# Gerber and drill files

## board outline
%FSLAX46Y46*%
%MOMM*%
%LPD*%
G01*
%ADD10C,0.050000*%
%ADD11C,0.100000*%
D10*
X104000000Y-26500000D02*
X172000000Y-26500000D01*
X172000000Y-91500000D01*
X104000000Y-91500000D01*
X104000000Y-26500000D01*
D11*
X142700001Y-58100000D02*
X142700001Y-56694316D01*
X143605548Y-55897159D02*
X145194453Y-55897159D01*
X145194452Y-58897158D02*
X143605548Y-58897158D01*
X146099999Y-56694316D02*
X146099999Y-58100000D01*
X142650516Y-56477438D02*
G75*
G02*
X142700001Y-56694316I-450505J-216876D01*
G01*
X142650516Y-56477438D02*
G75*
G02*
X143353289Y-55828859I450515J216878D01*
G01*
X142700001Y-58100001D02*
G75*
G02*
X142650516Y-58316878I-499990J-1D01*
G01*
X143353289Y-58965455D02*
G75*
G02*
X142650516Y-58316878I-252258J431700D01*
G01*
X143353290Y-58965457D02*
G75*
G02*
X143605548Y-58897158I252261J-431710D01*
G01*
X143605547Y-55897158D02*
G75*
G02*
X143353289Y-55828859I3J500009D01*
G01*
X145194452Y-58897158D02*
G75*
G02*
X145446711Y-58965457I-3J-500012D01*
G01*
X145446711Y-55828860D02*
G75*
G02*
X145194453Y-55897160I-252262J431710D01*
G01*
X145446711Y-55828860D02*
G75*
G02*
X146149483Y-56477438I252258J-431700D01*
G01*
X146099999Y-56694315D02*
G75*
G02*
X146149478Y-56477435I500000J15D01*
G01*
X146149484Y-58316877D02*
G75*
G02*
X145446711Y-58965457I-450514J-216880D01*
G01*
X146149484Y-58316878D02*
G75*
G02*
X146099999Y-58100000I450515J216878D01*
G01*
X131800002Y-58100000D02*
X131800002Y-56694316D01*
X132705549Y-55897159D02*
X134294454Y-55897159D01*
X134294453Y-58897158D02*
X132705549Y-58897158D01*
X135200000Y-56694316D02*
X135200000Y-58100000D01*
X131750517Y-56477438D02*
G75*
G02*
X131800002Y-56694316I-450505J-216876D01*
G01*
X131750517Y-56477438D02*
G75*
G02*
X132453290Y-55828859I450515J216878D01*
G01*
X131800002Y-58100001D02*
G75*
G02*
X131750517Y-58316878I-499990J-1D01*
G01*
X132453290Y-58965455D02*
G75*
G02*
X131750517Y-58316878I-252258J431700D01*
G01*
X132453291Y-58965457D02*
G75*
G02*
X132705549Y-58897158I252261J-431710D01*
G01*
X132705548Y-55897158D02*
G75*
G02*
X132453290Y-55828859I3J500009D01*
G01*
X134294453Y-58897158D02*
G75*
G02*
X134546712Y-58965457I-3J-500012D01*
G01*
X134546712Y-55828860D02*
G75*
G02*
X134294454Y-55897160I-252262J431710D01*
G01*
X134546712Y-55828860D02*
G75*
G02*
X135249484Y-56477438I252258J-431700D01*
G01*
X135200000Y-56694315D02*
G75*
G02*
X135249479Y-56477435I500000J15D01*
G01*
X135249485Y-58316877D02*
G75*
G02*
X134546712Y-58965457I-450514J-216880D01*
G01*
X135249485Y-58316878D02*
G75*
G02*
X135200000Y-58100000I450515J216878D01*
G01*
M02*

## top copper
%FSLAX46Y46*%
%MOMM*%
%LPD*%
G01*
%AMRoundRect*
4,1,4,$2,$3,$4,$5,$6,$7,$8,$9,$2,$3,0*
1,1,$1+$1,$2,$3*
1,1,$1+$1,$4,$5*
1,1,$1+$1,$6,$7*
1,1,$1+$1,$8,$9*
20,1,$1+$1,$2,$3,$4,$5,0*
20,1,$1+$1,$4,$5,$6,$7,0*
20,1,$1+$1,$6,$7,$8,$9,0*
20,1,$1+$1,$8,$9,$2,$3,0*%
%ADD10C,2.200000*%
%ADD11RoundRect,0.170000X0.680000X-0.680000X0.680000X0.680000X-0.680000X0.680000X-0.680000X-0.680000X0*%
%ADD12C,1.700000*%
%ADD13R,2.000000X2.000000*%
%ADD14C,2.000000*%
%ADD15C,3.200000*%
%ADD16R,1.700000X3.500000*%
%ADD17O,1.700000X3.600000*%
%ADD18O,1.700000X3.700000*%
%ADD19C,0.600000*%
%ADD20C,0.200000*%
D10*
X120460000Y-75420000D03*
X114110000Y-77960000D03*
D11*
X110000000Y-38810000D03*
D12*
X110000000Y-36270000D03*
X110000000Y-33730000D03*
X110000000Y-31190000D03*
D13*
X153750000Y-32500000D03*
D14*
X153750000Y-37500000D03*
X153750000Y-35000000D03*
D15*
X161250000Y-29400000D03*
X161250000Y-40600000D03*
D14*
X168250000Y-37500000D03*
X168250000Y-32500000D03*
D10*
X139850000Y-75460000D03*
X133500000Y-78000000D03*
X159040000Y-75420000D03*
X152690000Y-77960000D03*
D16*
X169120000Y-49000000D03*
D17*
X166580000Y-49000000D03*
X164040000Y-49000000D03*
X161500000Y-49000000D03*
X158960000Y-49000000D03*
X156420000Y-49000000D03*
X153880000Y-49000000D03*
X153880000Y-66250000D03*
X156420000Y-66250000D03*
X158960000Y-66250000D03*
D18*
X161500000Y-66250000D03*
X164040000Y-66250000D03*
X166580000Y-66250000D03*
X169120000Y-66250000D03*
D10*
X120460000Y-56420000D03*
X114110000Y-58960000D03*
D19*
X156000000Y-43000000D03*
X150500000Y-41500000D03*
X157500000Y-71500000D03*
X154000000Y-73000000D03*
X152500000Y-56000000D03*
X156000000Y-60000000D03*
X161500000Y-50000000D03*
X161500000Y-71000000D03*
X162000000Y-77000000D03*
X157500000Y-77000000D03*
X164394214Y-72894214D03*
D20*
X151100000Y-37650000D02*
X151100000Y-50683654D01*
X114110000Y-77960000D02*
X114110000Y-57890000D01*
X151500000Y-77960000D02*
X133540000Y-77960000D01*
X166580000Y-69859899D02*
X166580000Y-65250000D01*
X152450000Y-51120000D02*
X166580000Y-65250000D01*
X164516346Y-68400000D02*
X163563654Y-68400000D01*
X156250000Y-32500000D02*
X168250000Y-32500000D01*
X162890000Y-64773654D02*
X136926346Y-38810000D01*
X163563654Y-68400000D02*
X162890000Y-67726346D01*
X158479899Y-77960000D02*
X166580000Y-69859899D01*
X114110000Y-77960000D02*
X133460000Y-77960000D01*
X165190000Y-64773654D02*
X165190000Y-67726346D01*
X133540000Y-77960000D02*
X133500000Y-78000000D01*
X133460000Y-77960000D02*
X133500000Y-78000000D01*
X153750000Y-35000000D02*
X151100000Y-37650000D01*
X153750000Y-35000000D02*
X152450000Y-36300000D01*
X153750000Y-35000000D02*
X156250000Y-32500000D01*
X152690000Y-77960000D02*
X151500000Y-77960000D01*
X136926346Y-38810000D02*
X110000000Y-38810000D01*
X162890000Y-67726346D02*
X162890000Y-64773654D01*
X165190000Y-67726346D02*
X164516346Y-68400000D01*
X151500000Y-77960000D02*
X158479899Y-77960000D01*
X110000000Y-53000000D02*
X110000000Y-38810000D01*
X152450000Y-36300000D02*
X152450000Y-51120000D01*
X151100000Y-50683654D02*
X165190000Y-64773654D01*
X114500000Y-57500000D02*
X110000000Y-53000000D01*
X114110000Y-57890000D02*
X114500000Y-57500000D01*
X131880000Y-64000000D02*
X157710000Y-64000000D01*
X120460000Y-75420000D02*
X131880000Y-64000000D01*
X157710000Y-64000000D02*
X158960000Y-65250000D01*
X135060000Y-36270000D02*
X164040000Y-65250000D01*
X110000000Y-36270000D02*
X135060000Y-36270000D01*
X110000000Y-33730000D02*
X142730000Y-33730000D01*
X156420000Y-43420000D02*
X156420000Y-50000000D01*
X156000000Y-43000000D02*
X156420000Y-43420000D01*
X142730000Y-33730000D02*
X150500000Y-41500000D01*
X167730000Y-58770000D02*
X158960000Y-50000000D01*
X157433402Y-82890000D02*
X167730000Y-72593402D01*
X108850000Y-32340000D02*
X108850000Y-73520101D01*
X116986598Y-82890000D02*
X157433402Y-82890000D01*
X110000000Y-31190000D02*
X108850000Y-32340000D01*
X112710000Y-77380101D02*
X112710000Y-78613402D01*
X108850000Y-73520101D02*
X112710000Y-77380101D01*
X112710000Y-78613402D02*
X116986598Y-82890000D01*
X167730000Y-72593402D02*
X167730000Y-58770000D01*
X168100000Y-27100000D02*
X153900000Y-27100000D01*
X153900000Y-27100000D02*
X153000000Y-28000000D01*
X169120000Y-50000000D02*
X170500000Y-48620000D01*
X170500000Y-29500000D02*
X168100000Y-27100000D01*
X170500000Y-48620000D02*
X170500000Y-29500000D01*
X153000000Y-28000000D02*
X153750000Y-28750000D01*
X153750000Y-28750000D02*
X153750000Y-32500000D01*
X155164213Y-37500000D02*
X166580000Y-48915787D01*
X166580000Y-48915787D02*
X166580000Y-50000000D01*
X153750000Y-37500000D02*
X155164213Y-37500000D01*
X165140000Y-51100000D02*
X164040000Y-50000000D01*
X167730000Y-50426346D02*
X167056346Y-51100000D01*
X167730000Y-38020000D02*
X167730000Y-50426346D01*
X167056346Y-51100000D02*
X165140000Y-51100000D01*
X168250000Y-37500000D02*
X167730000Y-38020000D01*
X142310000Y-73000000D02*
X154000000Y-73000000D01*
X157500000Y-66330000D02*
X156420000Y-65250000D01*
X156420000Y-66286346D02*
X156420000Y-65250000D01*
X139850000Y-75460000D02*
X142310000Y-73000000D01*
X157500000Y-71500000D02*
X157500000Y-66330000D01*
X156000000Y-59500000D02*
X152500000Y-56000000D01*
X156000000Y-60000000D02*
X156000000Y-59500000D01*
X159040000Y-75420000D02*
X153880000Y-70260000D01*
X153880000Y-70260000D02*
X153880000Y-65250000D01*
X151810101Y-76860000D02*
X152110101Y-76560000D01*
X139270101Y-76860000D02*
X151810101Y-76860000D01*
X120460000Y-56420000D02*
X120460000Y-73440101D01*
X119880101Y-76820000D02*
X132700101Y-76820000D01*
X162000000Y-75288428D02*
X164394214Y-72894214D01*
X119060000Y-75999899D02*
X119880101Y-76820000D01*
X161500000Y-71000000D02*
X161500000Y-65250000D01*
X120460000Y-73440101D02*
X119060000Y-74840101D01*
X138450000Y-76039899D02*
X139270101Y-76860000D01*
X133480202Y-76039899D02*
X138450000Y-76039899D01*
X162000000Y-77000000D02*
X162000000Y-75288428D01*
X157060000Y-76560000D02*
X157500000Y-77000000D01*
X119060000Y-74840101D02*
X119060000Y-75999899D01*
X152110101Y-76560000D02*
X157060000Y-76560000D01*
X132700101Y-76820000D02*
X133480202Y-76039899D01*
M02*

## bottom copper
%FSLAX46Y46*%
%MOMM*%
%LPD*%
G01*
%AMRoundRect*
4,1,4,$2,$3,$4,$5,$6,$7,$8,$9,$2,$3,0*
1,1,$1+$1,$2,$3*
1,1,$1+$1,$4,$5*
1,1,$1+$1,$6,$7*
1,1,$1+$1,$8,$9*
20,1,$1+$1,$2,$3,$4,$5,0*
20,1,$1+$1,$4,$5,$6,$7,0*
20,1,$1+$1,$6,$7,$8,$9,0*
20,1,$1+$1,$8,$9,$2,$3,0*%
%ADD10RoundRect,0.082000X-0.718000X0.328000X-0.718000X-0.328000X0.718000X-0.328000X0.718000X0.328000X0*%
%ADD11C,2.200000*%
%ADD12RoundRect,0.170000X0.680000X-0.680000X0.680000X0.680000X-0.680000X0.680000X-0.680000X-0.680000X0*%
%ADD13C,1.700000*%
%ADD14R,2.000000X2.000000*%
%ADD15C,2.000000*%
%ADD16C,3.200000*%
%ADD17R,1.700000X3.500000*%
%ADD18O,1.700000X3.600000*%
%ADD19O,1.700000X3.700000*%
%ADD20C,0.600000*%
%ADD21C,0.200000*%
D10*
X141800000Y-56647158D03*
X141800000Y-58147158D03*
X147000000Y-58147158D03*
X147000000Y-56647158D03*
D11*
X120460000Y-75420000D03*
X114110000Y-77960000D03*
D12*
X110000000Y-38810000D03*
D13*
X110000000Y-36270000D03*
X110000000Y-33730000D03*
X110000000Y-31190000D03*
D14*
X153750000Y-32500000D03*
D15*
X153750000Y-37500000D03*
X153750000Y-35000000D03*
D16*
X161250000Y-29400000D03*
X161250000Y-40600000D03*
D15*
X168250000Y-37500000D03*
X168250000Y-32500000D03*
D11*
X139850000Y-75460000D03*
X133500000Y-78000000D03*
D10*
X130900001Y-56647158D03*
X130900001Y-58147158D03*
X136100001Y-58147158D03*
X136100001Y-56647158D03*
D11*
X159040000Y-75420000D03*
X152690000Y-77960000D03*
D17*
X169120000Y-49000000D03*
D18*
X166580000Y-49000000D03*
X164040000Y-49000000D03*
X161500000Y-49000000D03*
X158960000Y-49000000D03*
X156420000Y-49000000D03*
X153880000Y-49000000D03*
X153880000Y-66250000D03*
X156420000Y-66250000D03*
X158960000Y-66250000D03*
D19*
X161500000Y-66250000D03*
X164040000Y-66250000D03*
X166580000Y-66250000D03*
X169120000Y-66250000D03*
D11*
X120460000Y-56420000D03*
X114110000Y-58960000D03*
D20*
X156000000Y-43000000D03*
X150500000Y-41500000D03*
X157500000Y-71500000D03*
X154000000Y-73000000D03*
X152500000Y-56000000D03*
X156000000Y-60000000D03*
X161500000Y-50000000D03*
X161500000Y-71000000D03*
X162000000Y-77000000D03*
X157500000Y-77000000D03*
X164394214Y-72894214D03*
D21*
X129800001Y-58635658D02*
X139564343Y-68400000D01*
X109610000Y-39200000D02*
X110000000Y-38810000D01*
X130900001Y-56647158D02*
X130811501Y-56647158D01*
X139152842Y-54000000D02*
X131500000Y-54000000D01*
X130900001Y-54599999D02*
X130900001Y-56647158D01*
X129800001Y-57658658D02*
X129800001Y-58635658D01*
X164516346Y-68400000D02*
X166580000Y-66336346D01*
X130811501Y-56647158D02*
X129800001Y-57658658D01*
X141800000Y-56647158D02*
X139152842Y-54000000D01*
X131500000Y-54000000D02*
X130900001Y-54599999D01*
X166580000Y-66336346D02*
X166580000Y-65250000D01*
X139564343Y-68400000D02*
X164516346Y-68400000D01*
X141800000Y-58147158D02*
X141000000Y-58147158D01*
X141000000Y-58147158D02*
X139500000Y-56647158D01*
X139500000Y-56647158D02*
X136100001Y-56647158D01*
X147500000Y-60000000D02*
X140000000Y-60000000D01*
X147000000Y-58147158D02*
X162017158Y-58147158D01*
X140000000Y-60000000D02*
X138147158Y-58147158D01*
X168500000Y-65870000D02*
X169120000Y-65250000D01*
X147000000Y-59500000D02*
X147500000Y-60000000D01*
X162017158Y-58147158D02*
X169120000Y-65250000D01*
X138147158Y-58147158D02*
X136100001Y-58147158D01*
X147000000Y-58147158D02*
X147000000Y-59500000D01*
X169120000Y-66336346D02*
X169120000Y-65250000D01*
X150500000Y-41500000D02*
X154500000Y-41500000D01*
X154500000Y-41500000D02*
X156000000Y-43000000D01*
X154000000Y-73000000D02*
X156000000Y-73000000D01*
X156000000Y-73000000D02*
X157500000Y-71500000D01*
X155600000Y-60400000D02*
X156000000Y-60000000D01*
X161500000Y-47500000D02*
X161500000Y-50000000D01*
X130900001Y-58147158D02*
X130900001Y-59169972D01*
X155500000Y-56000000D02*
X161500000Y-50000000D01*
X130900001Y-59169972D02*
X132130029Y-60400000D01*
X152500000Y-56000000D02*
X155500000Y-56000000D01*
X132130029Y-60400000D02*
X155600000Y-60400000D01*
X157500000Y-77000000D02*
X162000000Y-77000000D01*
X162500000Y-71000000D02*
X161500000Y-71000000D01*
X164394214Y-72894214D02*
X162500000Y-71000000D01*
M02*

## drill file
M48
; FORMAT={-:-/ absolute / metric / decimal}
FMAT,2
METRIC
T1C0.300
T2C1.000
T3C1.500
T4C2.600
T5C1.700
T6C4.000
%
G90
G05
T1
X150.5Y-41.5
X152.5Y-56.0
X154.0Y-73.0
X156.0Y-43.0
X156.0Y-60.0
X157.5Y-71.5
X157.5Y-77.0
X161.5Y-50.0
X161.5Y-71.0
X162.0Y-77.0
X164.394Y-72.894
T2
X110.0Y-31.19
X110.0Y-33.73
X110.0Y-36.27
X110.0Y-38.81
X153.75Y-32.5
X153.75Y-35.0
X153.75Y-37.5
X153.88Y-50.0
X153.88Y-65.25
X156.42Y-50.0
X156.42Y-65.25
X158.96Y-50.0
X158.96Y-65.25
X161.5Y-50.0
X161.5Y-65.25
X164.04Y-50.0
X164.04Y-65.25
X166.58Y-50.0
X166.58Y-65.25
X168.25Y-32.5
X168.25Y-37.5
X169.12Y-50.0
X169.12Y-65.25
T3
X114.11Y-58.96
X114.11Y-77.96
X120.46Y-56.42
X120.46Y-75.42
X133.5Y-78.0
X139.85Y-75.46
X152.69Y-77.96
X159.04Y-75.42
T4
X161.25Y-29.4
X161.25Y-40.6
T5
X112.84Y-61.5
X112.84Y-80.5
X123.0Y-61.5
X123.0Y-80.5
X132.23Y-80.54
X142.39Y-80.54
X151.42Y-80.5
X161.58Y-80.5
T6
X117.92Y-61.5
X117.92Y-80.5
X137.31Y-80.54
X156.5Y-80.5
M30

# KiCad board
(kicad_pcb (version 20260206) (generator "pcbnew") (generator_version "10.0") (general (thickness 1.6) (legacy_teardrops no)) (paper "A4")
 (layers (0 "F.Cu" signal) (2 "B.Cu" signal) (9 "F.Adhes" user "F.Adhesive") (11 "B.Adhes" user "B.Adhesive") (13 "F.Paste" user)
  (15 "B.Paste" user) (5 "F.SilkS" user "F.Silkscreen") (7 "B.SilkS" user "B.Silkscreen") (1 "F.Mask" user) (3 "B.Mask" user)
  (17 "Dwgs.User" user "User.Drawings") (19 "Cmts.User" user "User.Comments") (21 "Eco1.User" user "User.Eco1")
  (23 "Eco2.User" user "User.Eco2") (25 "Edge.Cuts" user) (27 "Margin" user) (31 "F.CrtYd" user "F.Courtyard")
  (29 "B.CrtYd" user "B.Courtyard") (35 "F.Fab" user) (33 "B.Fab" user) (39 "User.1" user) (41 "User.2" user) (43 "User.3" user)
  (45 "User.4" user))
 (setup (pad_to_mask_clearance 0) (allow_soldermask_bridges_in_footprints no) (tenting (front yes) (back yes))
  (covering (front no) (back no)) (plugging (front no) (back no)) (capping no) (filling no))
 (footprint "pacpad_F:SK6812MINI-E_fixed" (layer "F.Cu") (at 144.399999 57.5)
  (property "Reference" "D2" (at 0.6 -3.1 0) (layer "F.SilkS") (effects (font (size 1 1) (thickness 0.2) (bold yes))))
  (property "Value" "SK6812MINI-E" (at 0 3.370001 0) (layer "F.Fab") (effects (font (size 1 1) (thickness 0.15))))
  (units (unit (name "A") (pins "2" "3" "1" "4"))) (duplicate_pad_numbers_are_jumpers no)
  (fp_line (start -1.699998 0.6) (end -1.699998 -0.805684) (stroke (width 0.1) (type solid)) (layer "Edge.Cuts"))
  (fp_line (start -0.794451 -1.602841) (end 0.794454 -1.602841) (stroke (width 0.1) (type solid)) (layer "Edge.Cuts"))
  (fp_line (start 0.794453 1.397158) (end -0.794451 1.397158) (stroke (width 0.1) (type solid)) (layer "Edge.Cuts"))
  (fp_line (start 1.7 -0.805684) (end 1.7 0.6) (stroke (width 0.1) (type solid)) (layer "Edge.Cuts"))
  (fp_arc (start -1.749483 -1.022562) (mid -1.712526 -0.91691) (end -1.699998 -0.805684) (stroke (width 0.1) (type solid))
   (layer "Edge.Cuts"))
  (fp_arc (start -1.749483 -1.022562) (mid -1.63807 -1.606877) (end -1.04671 -1.671141) (stroke (width 0.1) (type solid))
   (layer "Edge.Cuts"))
  (fp_arc (start -1.699998 0.600001) (mid -1.712526 0.711226) (end -1.749483 0.816878) (stroke (width 0.1) (type solid)) (layer "Edge.Cuts"))
  (fp_arc (start -1.04671 1.465455) (mid -1.638069 1.401192) (end -1.749483 0.816878) (stroke (width 0.1) (type solid)) (layer "Edge.Cuts"))
  (fp_arc (start -1.046709 1.465457) (mid -0.925121 1.414535) (end -0.794451 1.397158) (stroke (width 0.1) (type solid)) (layer "Edge.Cuts"))
  (fp_arc (start -0.794452 -1.602842) (mid -0.925122 -1.620219) (end -1.04671 -1.671141) (stroke (width 0.1) (type solid))
   (layer "Edge.Cuts"))
  (fp_arc (start 0.794453 1.397158) (mid 0.925124 1.414535) (end 1.046712 1.465457) (stroke (width 0.1) (type solid)) (layer "Edge.Cuts"))
  (fp_arc (start 1.046712 -1.67114) (mid 0.925124 -1.620218) (end 0.794454 -1.602841) (stroke (width 0.1) (type solid)) (layer "Edge.Cuts"))
  (fp_arc (start 1.046712 -1.67114) (mid 1.638072 -1.606876) (end 1.749485 -1.022562) (stroke (width 0.1) (type solid)) (layer "Edge.Cuts"))
  (fp_arc (start 1.7 -0.805685) (mid 1.712528 -0.91691) (end 1.749485 -1.022562) (stroke (width 0.1) (type solid)) (layer "Edge.Cuts"))
  (fp_arc (start 1.749485 0.816877) (mid 1.638073 1.401193) (end 1.046712 1.465457) (stroke (width 0.1) (type solid)) (layer "Edge.Cuts"))
  (fp_arc (start 1.749485 0.816878) (mid 1.712528 0.711226) (end 1.7 0.6) (stroke (width 0.1) (type solid)) (layer "Edge.Cuts"))
  (pad "1" smd roundrect (at -2.599999 -0.852842 270) (size 0.82 1.6) (layers "B.Cu" "B.Mask" "B.Paste") (roundrect_rratio 0.1) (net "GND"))
  (pad "2" smd roundrect (at -2.599999 0.647158 270) (size 0.82 1.6) (layers "B.Cu" "B.Mask" "B.Paste") (roundrect_rratio 0.1)
   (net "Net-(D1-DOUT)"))
  (pad "3" smd roundrect (at 2.600001 0.647158 270) (size 0.82 1.6) (layers "B.Cu" "B.Mask" "B.Paste") (roundrect_rratio 0.1)
   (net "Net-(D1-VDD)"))
  (pad "4" smd roundrect (at 2.600001 -0.852842 270) (size 0.82 1.6) (layers "B.Cu" "B.Mask" "B.Paste") (roundrect_rratio 0.1)
   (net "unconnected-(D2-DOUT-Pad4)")))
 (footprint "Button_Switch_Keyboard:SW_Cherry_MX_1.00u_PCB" (layer "F.Cu") (at 120.46 75.42)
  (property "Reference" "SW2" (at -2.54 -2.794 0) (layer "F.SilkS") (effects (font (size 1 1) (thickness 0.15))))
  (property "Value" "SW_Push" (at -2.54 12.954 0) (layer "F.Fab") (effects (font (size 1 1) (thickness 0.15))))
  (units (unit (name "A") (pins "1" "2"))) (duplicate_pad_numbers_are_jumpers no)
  (pad "" np_thru_hole circle (at -7.62 5.08) (size 1.7 1.7) (drill 1.7) (layers "*.Cu" "*.Mask"))
  (pad "" np_thru_hole circle (at -2.54 5.08) (size 4 4) (drill 4) (layers "*.Cu" "*.Mask"))
  (pad "" np_thru_hole circle (at 2.54 5.08) (size 1.7 1.7) (drill 1.7) (layers "*.Cu" "*.Mask"))
  (pad "1" thru_hole circle (at 0 0) (size 2.2 2.2) (drill 1.5) (layers "*.Cu" "*.Mask") (remove_unused_layers no)
   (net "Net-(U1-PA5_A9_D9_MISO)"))
  (pad "2" thru_hole circle (at -6.35 2.54) (size 2.2 2.2) (drill 1.5) (layers "*.Cu" "*.Mask") (remove_unused_layers no) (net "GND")))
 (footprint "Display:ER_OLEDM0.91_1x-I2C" (layer "F.Cu") (at 110 38.81 90)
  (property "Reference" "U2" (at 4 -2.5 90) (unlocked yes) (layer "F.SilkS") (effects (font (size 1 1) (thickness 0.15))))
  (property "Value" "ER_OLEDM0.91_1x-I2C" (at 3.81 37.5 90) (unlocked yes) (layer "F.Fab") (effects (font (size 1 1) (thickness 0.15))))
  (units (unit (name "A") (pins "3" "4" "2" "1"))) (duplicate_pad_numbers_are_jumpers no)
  (pad "1" thru_hole roundrect (at 0 0 90) (size 1.7 1.7) (drill 1) (layers "*.Cu" "*.Mask") (remove_unused_layers no)
   (roundrect_rratio 0.1) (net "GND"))
  (pad "2" thru_hole circle (at 2.54 0 90) (size 1.7 1.7) (drill 1) (layers "*.Cu" "*.Mask") (remove_unused_layers no) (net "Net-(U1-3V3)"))
  (pad "3" thru_hole circle (at 5.08 0 90) (size 1.7 1.7) (drill 1) (layers "*.Cu" "*.Mask") (remove_unused_layers no)
   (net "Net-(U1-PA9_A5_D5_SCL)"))
  (pad "4" thru_hole circle (at 7.62 0 90) (size 1.7 1.7) (drill 1) (layers "*.Cu" "*.Mask") (remove_unused_layers no)
   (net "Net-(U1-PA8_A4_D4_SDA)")))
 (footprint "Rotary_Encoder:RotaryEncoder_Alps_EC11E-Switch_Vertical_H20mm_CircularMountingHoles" (layer "F.Cu") (at 153.75 32.5)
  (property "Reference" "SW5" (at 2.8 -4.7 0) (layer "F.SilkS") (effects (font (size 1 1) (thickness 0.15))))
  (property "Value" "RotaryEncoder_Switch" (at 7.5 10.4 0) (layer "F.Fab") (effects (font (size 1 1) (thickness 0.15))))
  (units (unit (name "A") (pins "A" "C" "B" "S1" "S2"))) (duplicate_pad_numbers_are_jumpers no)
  (pad "A" thru_hole rect (at 0 0) (size 2 2) (drill 1) (layers "*.Cu" "*.Mask") (remove_unused_layers no) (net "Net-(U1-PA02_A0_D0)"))
  (pad "B" thru_hole circle (at 0 5) (size 2 2) (drill 1) (layers "*.Cu" "*.Mask") (remove_unused_layers no) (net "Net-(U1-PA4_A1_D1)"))
  (pad "C" thru_hole circle (at 0 2.5) (size 2 2) (drill 1) (layers "*.Cu" "*.Mask") (remove_unused_layers no) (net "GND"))
  (pad "MP" thru_hole circle (at 7.5 -3.1) (size 3.2 3.2) (drill 2.6) (layers "*.Cu" "*.Mask") (remove_unused_layers no))
  (pad "MP" thru_hole circle (at 7.5 8.1) (size 3.2 3.2) (drill 2.6) (layers "*.Cu" "*.Mask") (remove_unused_layers no))
  (pad "S1" thru_hole circle (at 14.5 5) (size 2 2) (drill 1) (layers "*.Cu" "*.Mask") (remove_unused_layers no) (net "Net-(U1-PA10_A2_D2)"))
  (pad "S2" thru_hole circle (at 14.5 0) (size 2 2) (drill 1) (layers "*.Cu" "*.Mask") (remove_unused_layers no) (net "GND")))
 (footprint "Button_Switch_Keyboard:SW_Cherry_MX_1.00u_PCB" (layer "F.Cu") (at 139.85 75.46)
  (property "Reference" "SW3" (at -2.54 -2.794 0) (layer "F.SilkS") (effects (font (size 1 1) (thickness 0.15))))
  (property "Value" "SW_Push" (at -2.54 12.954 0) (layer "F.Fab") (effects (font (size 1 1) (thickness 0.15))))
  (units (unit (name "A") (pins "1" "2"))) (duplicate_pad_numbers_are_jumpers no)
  (pad "" np_thru_hole circle (at -7.62 5.08) (size 1.7 1.7) (drill 1.7) (layers "*.Cu" "*.Mask"))
  (pad "" np_thru_hole circle (at -2.54 5.08) (size 4 4) (drill 4) (layers "*.Cu" "*.Mask"))
  (pad "" np_thru_hole circle (at 2.54 5.08) (size 1.7 1.7) (drill 1.7) (layers "*.Cu" "*.Mask"))
  (pad "1" thru_hole circle (at 0 0) (size 2.2 2.2) (drill 1.5) (layers "*.Cu" "*.Mask") (remove_unused_layers no)
   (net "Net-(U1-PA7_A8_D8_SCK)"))
  (pad "2" thru_hole circle (at -6.35 2.54) (size 2.2 2.2) (drill 1.5) (layers "*.Cu" "*.Mask") (remove_unused_layers no) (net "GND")))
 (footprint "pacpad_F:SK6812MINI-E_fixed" (layer "F.Cu") (at 133.5 57.5)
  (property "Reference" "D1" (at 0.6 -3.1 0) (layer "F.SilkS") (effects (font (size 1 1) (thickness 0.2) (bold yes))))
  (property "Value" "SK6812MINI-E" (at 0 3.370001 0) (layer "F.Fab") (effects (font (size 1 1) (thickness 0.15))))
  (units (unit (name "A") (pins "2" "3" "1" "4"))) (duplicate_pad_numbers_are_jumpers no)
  (fp_line (start -1.699998 0.6) (end -1.699998 -0.805684) (stroke (width 0.1) (type solid)) (layer "Edge.Cuts"))
  (fp_line (start -0.794451 -1.602841) (end 0.794454 -1.602841) (stroke (width 0.1) (type solid)) (layer "Edge.Cuts"))
  (fp_line (start 0.794453 1.397158) (end -0.794451 1.397158) (stroke (width 0.1) (type solid)) (layer "Edge.Cuts"))
  (fp_line (start 1.7 -0.805684) (end 1.7 0.6) (stroke (width 0.1) (type solid)) (layer "Edge.Cuts"))
  (fp_arc (start -1.749483 -1.022562) (mid -1.712526 -0.91691) (end -1.699998 -0.805684) (stroke (width 0.1) (type solid))
   (layer "Edge.Cuts"))
  (fp_arc (start -1.749483 -1.022562) (mid -1.63807 -1.606877) (end -1.04671 -1.671141) (stroke (width 0.1) (type solid))
   (layer "Edge.Cuts"))
  (fp_arc (start -1.699998 0.600001) (mid -1.712526 0.711226) (end -1.749483 0.816878) (stroke (width 0.1) (type solid)) (layer "Edge.Cuts"))
  (fp_arc (start -1.04671 1.465455) (mid -1.638069 1.401192) (end -1.749483 0.816878) (stroke (width 0.1) (type solid)) (layer "Edge.Cuts"))
  (fp_arc (start -1.046709 1.465457) (mid -0.925121 1.414535) (end -0.794451 1.397158) (stroke (width 0.1) (type solid)) (layer "Edge.Cuts"))
  (fp_arc (start -0.794452 -1.602842) (mid -0.925122 -1.620219) (end -1.04671 -1.671141) (stroke (width 0.1) (type solid))
   (layer "Edge.Cuts"))
  (fp_arc (start 0.794453 1.397158) (mid 0.925124 1.414535) (end 1.046712 1.465457) (stroke (width 0.1) (type solid)) (layer "Edge.Cuts"))
  (fp_arc (start 1.046712 -1.67114) (mid 0.925124 -1.620218) (end 0.794454 -1.602841) (stroke (width 0.1) (type solid)) (layer "Edge.Cuts"))
  (fp_arc (start 1.046712 -1.67114) (mid 1.638072 -1.606876) (end 1.749485 -1.022562) (stroke (width 0.1) (type solid)) (layer "Edge.Cuts"))
  (fp_arc (start 1.7 -0.805685) (mid 1.712528 -0.91691) (end 1.749485 -1.022562) (stroke (width 0.1) (type solid)) (layer "Edge.Cuts"))
  (fp_arc (start 1.749485 0.816877) (mid 1.638073 1.401193) (end 1.046712 1.465457) (stroke (width 0.1) (type solid)) (layer "Edge.Cuts"))
  (fp_arc (start 1.749485 0.816878) (mid 1.712528 0.711226) (end 1.7 0.6) (stroke (width 0.1) (type solid)) (layer "Edge.Cuts"))
  (pad "1" smd roundrect (at -2.599999 -0.852842 270) (size 0.82 1.6) (layers "B.Cu" "B.Mask" "B.Paste") (roundrect_rratio 0.1) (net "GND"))
  (pad "2" smd roundrect (at -2.599999 0.647158 270) (size 0.82 1.6) (layers "B.Cu" "B.Mask" "B.Paste") (roundrect_rratio 0.1)
   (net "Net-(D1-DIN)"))
  (pad "3" smd roundrect (at 2.600001 0.647158 270) (size 0.82 1.6) (layers "B.Cu" "B.Mask" "B.Paste") (roundrect_rratio 0.1)
   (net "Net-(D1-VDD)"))
  (pad "4" smd roundrect (at 2.600001 -0.852842 270) (size 0.82 1.6) (layers "B.Cu" "B.Mask" "B.Paste") (roundrect_rratio 0.1)
   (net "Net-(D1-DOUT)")))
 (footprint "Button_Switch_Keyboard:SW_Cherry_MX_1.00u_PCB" (layer "F.Cu") (at 159.04 75.42)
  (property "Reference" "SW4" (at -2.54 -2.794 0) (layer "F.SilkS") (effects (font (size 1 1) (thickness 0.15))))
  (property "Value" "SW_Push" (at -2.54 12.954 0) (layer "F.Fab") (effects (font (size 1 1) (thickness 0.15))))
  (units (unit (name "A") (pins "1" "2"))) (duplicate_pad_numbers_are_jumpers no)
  (pad "" np_thru_hole circle (at -7.62 5.08) (size 1.7 1.7) (drill 1.7) (layers "*.Cu" "*.Mask"))
  (pad "" np_thru_hole circle (at -2.54 5.08) (size 4 4) (drill 4) (layers "*.Cu" "*.Mask"))
  (pad "" np_thru_hole circle (at 2.54 5.08) (size 1.7 1.7) (drill 1.7) (layers "*.Cu" "*.Mask"))
  (pad "1" thru_hole circle (at 0 0) (size 2.2 2.2) (drill 1.5) (layers "*.Cu" "*.Mask") (remove_unused_layers no)
   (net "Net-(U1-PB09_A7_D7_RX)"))
  (pad "2" thru_hole circle (at -6.35 2.54) (size 2.2 2.2) (drill 1.5) (layers "*.Cu" "*.Mask") (remove_unused_layers no) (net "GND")))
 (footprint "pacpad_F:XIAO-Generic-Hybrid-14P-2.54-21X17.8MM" (layer "F.Cu") (at 161.5 57.625 -90)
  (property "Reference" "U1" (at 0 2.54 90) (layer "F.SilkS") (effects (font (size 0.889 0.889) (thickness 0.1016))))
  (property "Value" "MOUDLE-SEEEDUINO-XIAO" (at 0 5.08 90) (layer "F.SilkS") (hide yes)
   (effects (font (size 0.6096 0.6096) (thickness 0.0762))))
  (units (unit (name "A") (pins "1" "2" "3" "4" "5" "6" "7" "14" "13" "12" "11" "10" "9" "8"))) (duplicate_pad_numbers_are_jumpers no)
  (pad "1" thru_hole rect (at -7.625 -7.62 270) (size 3.5 1.7) (drill 1 (offset -1 0)) (layers "*.Cu" "*.Mask") (remove_unused_layers no)
   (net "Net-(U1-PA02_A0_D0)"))
  (pad "2" thru_hole oval (at -7.625 -5.08 270) (size 3.6 1.7) (drill 1 (offset -1 0)) (layers "*.Cu" "*.Mask") (remove_unused_layers no)
   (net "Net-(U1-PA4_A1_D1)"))
  (pad "3" thru_hole oval (at -7.625 -2.54 270) (size 3.6 1.7) (drill 1 (offset -1 0)) (layers "*.Cu" "*.Mask") (remove_unused_layers no)
   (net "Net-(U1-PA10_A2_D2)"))
  (pad "4" thru_hole oval (at -7.625 0 270) (size 3.6 1.7) (drill 1 (offset -1 0)) (layers "*.Cu" "*.Mask") (remove_unused_layers no)
   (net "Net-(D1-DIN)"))
  (pad "5" thru_hole oval (at -7.625 2.54 270) (size 3.6 1.7) (drill 1 (offset -1 0)) (layers "*.Cu" "*.Mask") (remove_unused_layers no)
   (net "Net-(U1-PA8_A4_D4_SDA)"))
  (pad "6" thru_hole oval (at -7.625 5.08 90) (size 3.6 1.7) (drill 1 (offset 1 0)) (layers "*.Cu" "*.Mask") (remove_unused_layers no)
   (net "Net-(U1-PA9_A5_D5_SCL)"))
  (pad "7" thru_hole oval (at -7.625 7.62 270) (size 3.6 1.7) (drill 1 (offset -1 0)) (layers "*.Cu" "*.Mask") (remove_unused_layers no)
   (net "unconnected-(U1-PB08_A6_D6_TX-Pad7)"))
  (pad "8" thru_hole oval (at 7.625 7.62 270) (size 3.6 1.7) (drill 1 (offset 1 0)) (layers "*.Cu" "*.Mask") (remove_unused_layers no)
   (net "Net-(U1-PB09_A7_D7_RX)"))
  (pad "9" thru_hole oval (at 7.625 5.08 270) (size 3.6 1.7) (drill 1 (offset 1 0)) (layers "*.Cu" "*.Mask") (remove_unused_layers no)
   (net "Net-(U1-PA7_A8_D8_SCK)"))
  (pad "10" thru_hole oval (at 7.625 2.54 270) (size 3.6 1.7) (drill 1 (offset 1 0)) (layers "*.Cu" "*.Mask") (remove_unused_layers no)
   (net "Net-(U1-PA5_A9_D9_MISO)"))
  (pad "11" thru_hole oval (at 7.625 0 270) (size 3.7 1.7) (drill 1 (offset 1 0)) (layers "*.Cu" "*.Mask") (remove_unused_layers no)
   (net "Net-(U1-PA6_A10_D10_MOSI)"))
  (pad "12" thru_hole oval (at 7.625 -2.54 270) (size 3.7 1.7) (drill 1 (offset 1 0)) (layers "*.Cu" "*.Mask") (remove_unused_layers no)
   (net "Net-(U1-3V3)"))
  (pad "13" thru_hole oval (at 7.625 -5.08 270) (size 3.7 1.7) (drill 1 (offset 1 0)) (layers "*.Cu" "*.Mask") (remove_unused_layers no)
   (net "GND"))
  (pad "14" thru_hole oval (at 7.625 -7.62 270) (size 3.7 1.7) (drill 1 (offset 1 0)) (layers "*.Cu" "*.Mask") (remove_unused_layers no)
   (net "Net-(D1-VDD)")))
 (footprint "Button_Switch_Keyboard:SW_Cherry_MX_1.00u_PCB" (layer "F.Cu") (at 120.46 56.42)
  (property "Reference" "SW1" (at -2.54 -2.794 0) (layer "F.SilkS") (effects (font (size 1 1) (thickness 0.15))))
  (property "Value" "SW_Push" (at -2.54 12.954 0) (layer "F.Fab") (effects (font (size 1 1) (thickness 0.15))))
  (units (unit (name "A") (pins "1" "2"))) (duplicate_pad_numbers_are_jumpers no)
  (pad "" np_thru_hole circle (at -7.62 5.08) (size 1.7 1.7) (drill 1.7) (layers "*.Cu" "*.Mask"))
  (pad "" np_thru_hole circle (at -2.54 5.08) (size 4 4) (drill 4) (layers "*.Cu" "*.Mask"))
  (pad "" np_thru_hole circle (at 2.54 5.08) (size 1.7 1.7) (drill 1.7) (layers "*.Cu" "*.Mask"))
  (pad "1" thru_hole circle (at 0 0) (size 2.2 2.2) (drill 1.5) (layers "*.Cu" "*.Mask") (remove_unused_layers no)
   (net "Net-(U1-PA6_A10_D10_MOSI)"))
  (pad "2" thru_hole circle (at -6.35 2.54) (size 2.2 2.2) (drill 1.5) (layers "*.Cu" "*.Mask") (remove_unused_layers no) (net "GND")))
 (gr_rect (start 104 26.5) (end 172 91.5) (stroke (width 0.05) (type default)) (fill no) (layer "Edge.Cuts"))
 (segment (start 151.1 37.65) (end 151.1 50.683654) (width 0.2) (layer "F.Cu") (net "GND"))
 (segment (start 114.11 77.96) (end 114.11 57.89) (width 0.2) (layer "F.Cu") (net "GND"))
 (segment (start 151.5 77.96) (end 133.54 77.96) (width 0.2) (layer "F.Cu") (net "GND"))
 (segment (start 166.58 69.859899) (end 166.58 65.25) (width 0.2) (layer "F.Cu") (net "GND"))
 (segment (start 152.45 51.12) (end 166.58 65.25) (width 0.2) (layer "F.Cu") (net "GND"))
 (segment (start 164.516346 68.4) (end 163.563654 68.4) (width 0.2) (layer "F.Cu") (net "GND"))
 (segment (start 156.25 32.5) (end 168.25 32.5) (width 0.2) (layer "F.Cu") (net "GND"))
 (segment (start 162.89 64.773654) (end 136.926346 38.81) (width 0.2) (layer "F.Cu") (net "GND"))
 (segment (start 163.563654 68.4) (end 162.89 67.726346) (width 0.2) (layer "F.Cu") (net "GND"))
 (segment (start 158.479899 77.96) (end 166.58 69.859899) (width 0.2) (layer "F.Cu") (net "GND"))
 (segment (start 114.11 77.96) (end 133.46 77.96) (width 0.2) (layer "F.Cu") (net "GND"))
 (segment (start 165.19 64.773654) (end 165.19 67.726346) (width 0.2) (layer "F.Cu") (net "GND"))
 (segment (start 133.54 77.96) (end 133.5 78) (width 0.2) (layer "F.Cu") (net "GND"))
 (segment (start 133.46 77.96) (end 133.5 78) (width 0.2) (layer "F.Cu") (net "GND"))
 (segment (start 153.75 35) (end 151.1 37.65) (width 0.2) (layer "F.Cu") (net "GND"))
 (segment (start 153.75 35) (end 152.45 36.3) (width 0.2) (layer "F.Cu") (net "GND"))
 (segment (start 153.75 35) (end 156.25 32.5) (width 0.2) (layer "F.Cu") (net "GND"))
 (segment (start 152.69 77.96) (end 151.5 77.96) (width 0.2) (layer "F.Cu") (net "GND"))
 (segment (start 136.926346 38.81) (end 110 38.81) (width 0.2) (layer "F.Cu") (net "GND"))
 (segment (start 162.89 67.726346) (end 162.89 64.773654) (width 0.2) (layer "F.Cu") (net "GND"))
 (segment (start 165.19 67.726346) (end 164.516346 68.4) (width 0.2) (layer "F.Cu") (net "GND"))
 (segment (start 151.5 77.96) (end 158.479899 77.96) (width 0.2) (layer "F.Cu") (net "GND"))
 (segment (start 110 53) (end 110 38.81) (width 0.2) (layer "F.Cu") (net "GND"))
 (segment (start 152.45 36.3) (end 152.45 51.12) (width 0.2) (layer "F.Cu") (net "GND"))
 (segment (start 151.1 50.683654) (end 165.19 64.773654) (width 0.2) (layer "F.Cu") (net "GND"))
 (segment (start 114.5 57.5) (end 110 53) (width 0.2) (layer "F.Cu") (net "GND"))
 (segment (start 114.11 57.89) (end 114.5 57.5) (width 0.2) (layer "F.Cu") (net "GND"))
 (segment (start 129.800001 58.635658) (end 139.564343 68.4) (width 0.2) (layer "B.Cu") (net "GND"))
 (segment (start 109.61 39.2) (end 110 38.81) (width 0.2) (layer "B.Cu") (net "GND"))
 (segment (start 130.900001 56.647158) (end 130.811501 56.647158) (width 0.2) (layer "B.Cu") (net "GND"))
 (segment (start 139.152842 54) (end 131.5 54) (width 0.2) (layer "B.Cu") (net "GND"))
 (segment (start 130.900001 54.599999) (end 130.900001 56.647158) (width 0.2) (layer "B.Cu") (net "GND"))
 (segment (start 129.800001 57.658658) (end 129.800001 58.635658) (width 0.2) (layer "B.Cu") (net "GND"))
 (segment (start 164.516346 68.4) (end 166.58 66.336346) (width 0.2) (layer "B.Cu") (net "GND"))
 (segment (start 130.811501 56.647158) (end 129.800001 57.658658) (width 0.2) (layer "B.Cu") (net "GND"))
 (segment (start 141.8 56.647158) (end 139.152842 54) (width 0.2) (layer "B.Cu") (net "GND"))
 (segment (start 131.5 54) (end 130.900001 54.599999) (width 0.2) (layer "B.Cu") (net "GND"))
 (segment (start 166.58 66.336346) (end 166.58 65.25) (width 0.2) (layer "B.Cu") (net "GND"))
 (segment (start 139.564343 68.4) (end 164.516346 68.4) (width 0.2) (layer "B.Cu") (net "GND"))
 (segment (start 141.8 58.147158) (end 141 58.147158) (width 0.2) (layer "B.Cu") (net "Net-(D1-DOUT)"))
 (segment (start 141 58.147158) (end 139.5 56.647158) (width 0.2) (layer "B.Cu") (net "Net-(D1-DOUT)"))
 (segment (start 139.5 56.647158) (end 136.100001 56.647158) (width 0.2) (layer "B.Cu") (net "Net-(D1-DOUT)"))
 (segment (start 147.5 60) (end 140 60) (width 0.2) (layer "B.Cu") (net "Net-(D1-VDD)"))
 (segment (start 147 58.147158) (end 162.017158 58.147158) (width 0.2) (layer "B.Cu") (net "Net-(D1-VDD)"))
 (segment (start 140 60) (end 138.147158 58.147158) (width 0.2) (layer "B.Cu") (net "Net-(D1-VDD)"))
 (segment (start 168.5 65.87) (end 169.12 65.25) (width 0.2) (layer "B.Cu") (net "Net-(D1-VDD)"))
 (segment (start 147 59.5) (end 147.5 60) (width 0.2) (layer "B.Cu") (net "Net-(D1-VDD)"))
 (segment (start 162.017158 58.147158) (end 169.12 65.25) (width 0.2) (layer "B.Cu") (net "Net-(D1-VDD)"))
 (segment (start 138.147158 58.147158) (end 136.100001 58.147158) (width 0.2) (layer "B.Cu") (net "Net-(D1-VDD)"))
 (segment (start 147 58.147158) (end 147 59.5) (width 0.2) (layer "B.Cu") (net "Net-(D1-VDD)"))
 (segment (start 169.12 66.336346) (end 169.12 65.25) (width 0.2) (layer "B.Cu") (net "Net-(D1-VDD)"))
 (segment (start 131.88 64) (end 157.71 64) (width 0.2) (layer "F.Cu") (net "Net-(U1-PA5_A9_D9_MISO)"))
 (segment (start 120.46 75.42) (end 131.88 64) (width 0.2) (layer "F.Cu") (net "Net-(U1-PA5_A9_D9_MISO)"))
 (segment (start 157.71 64) (end 158.96 65.25) (width 0.2) (layer "F.Cu") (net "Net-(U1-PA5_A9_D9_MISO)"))
 (segment (start 135.06 36.27) (end 164.04 65.25) (width 0.2) (layer "F.Cu") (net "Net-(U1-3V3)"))
 (segment (start 110 36.27) (end 135.06 36.27) (width 0.2) (layer "F.Cu") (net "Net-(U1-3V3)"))
 (segment (start 110 33.73) (end 142.73 33.73) (width 0.2) (layer "F.Cu") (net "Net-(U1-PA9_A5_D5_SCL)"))
 (segment (start 156.42 43.42) (end 156.42 50) (width 0.2) (layer "F.Cu") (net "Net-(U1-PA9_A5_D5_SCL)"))
 (segment (start 156 43) (end 156.42 43.42) (width 0.2) (layer "F.Cu") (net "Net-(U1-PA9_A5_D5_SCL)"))
 (segment (start 142.73 33.73) (end 150.5 41.5) (width 0.2) (layer "F.Cu") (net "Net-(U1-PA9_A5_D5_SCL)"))
 (via (at 156 43) (size 0.6) (drill 0.3) (layers "F.Cu" "B.Cu") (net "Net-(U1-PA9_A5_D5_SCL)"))
 (via (at 150.5 41.5) (size 0.6) (drill 0.3) (layers "F.Cu" "B.Cu") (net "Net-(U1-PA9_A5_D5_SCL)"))
 (segment (start 150.5 41.5) (end 154.5 41.5) (width 0.2) (layer "B.Cu") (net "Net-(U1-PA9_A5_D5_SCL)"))
 (segment (start 154.5 41.5) (end 156 43) (width 0.2) (layer "B.Cu") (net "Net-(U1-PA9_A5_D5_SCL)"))
 (segment (start 167.73 58.77) (end 158.96 50) (width 0.2) (layer "F.Cu") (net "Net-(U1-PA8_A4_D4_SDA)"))
 (segment (start 157.433402 82.89) (end 167.73 72.593402) (width 0.2) (layer "F.Cu") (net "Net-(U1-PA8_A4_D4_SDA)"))
 (segment (start 108.85 32.34) (end 108.85 73.520101) (width 0.2) (layer "F.Cu") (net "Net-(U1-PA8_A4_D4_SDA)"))
 (segment (start 116.986598 82.89) (end 157.433402 82.89) (width 0.2) (layer "F.Cu") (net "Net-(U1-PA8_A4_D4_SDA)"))
 (segment (start 110 31.19) (end 108.85 32.34) (width 0.2) (layer "F.Cu") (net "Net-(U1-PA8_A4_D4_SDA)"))
 (segment (start 112.71 77.380101) (end 112.71 78.613402) (width 0.2) (layer "F.Cu") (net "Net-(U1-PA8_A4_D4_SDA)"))
 (segment (start 108.85 73.520101) (end 112.71 77.380101) (width 0.2) (layer "F.Cu") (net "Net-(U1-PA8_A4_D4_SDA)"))
 (segment (start 112.71 78.613402) (end 116.986598 82.89) (width 0.2) (layer "F.Cu") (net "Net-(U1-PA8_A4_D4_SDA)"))
 (segment (start 167.73 72.593402) (end 167.73 58.77) (width 0.2) (layer "F.Cu") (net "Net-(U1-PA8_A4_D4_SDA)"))
 (segment (start 168.1 27.1) (end 153.9 27.1) (width 0.2) (layer "F.Cu") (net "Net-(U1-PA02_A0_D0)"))
 (segment (start 153.9 27.1) (end 153 28) (width 0.2) (layer "F.Cu") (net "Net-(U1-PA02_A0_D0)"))
 (segment (start 169.12 50) (end 170.5 48.62) (width 0.2) (layer "F.Cu") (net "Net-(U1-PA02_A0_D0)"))
 (segment (start 170.5 29.5) (end 168.1 27.1) (width 0.2) (layer "F.Cu") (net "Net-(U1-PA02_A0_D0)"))
 (segment (start 170.5 48.62) (end 170.5 29.5) (width 0.2) (layer "F.Cu") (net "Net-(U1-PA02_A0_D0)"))
 (segment (start 153 28) (end 153.75 28.75) (width 0.2) (layer "F.Cu") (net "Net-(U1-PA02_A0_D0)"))
 (segment (start 153.75 28.75) (end 153.75 32.5) (width 0.2) (layer "F.Cu") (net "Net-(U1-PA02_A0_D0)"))
 (segment (start 155.164213 37.5) (end 166.58 48.915787) (width 0.2) (layer "F.Cu") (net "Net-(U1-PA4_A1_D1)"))
 (segment (start 166.58 48.915787) (end 166.58 50) (width 0.2) (layer "F.Cu") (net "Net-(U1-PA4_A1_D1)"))
 (segment (start 153.75 37.5) (end 155.164213 37.5) (width 0.2) (layer "F.Cu") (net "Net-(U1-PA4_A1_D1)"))
 (segment (start 165.14 51.1) (end 164.04 50) (width 0.2) (layer "F.Cu") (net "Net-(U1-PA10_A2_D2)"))
 (segment (start 167.73 50.426346) (end 167.056346 51.1) (width 0.2) (layer "F.Cu") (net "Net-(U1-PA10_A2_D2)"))
 (segment (start 167.73 38.02) (end 167.73 50.426346) (width 0.2) (layer "F.Cu") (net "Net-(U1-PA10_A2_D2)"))
 (segment (start 167.056346 51.1) (end 165.14 51.1) (width 0.2) (layer "F.Cu") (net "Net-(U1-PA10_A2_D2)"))
 (segment (start 168.25 37.5) (end 167.73 38.02) (width 0.2) (layer "F.Cu") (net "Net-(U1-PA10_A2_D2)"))
 (segment (start 142.31 73) (end 154 73) (width 0.2) (layer "F.Cu") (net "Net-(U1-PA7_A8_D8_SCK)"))
 (segment (start 157.5 66.33) (end 156.42 65.25) (width 0.2) (layer "F.Cu") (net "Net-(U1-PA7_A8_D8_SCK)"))
 (segment (start 156.42 66.286346) (end 156.42 65.25) (width 0.2) (layer "F.Cu") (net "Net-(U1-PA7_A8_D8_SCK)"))
 (segment (start 139.85 75.46) (end 142.31 73) (width 0.2) (layer "F.Cu") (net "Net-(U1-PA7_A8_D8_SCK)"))
 (segment (start 157.5 71.5) (end 157.5 66.33) (width 0.2) (layer "F.Cu") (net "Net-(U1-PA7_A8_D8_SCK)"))
 (via (at 157.5 71.5) (size 0.6) (drill 0.3) (layers "F.Cu" "B.Cu") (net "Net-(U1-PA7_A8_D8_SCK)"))
 (via (at 154 73) (size 0.6) (drill 0.3) (layers "F.Cu" "B.Cu") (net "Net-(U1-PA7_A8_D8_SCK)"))
 (segment (start 154 73) (end 156 73) (width 0.2) (layer "B.Cu") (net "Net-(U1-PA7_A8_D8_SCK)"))
 (segment (start 156 73) (end 157.5 71.5) (width 0.2) (layer "B.Cu") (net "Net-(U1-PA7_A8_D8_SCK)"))
 (segment (start 156 59.5) (end 152.5 56) (width 0.2) (layer "F.Cu") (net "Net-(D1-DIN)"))
 (segment (start 156 60) (end 156 59.5) (width 0.2) (layer "F.Cu") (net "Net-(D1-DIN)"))
 (via (at 152.5 56) (size 0.6) (drill 0.3) (layers "F.Cu" "B.Cu") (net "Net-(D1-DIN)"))
 (via (at 156 60) (size 0.6) (drill 0.3) (layers "F.Cu" "B.Cu") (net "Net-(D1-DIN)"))
 (via (at 161.5 50) (size 0.6) (drill 0.3) (layers "F.Cu" "B.Cu") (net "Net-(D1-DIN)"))
 (segment (start 155.6 60.4) (end 156 60) (width 0.2) (layer "B.Cu") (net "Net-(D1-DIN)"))
 (segment (start 161.5 47.5) (end 161.5 50) (width 0.2) (layer "B.Cu") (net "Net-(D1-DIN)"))
 (segment (start 130.900001 58.147158) (end 130.900001 59.169972) (width 0.2) (layer "B.Cu") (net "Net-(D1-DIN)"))
 (segment (start 155.5 56) (end 161.5 50) (width 0.2) (layer "B.Cu") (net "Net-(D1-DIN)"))
 (segment (start 130.900001 59.169972) (end 132.130029 60.4) (width 0.2) (layer "B.Cu") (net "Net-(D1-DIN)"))
 (segment (start 152.5 56) (end 155.5 56) (width 0.2) (layer "B.Cu") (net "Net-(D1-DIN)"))
 (segment (start 132.130029 60.4) (end 155.6 60.4) (width 0.2) (layer "B.Cu") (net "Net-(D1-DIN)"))
 (segment (start 159.04 75.42) (end 153.88 70.26) (width 0.2) (layer "F.Cu") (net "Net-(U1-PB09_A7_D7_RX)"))
 (segment (start 153.88 70.26) (end 153.88 65.25) (width 0.2) (layer "F.Cu") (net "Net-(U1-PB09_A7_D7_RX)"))
 (segment (start 151.810101 76.86) (end 152.110101 76.56) (width 0.2) (layer "F.Cu") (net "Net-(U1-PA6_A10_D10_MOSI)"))
 (segment (start 139.270101 76.86) (end 151.810101 76.86) (width 0.2) (layer "F.Cu") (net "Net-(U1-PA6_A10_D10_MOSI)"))
 (segment (start 120.46 56.42) (end 120.46 73.440101) (width 0.2) (layer "F.Cu") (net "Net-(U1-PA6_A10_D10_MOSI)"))
 (segment (start 119.880101 76.82) (end 132.700101 76.82) (width 0.2) (layer "F.Cu") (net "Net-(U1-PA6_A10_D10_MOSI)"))
 (segment (start 162 75.288428) (end 164.394214 72.894214) (width 0.2) (layer "F.Cu") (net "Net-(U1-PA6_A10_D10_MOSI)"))
 (segment (start 119.06 75.999899) (end 119.880101 76.82) (width 0.2) (layer "F.Cu") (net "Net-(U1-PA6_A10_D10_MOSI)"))
 (segment (start 161.5 71) (end 161.5 65.25) (width 0.2) (layer "F.Cu") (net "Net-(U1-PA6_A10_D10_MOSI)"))
 (segment (start 120.46 73.440101) (end 119.06 74.840101) (width 0.2) (layer "F.Cu") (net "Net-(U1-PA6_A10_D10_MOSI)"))
 (segment (start 138.45 76.039899) (end 139.270101 76.86) (width 0.2) (layer "F.Cu") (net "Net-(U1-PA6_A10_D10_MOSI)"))
 (segment (start 133.480202 76.039899) (end 138.45 76.039899) (width 0.2) (layer "F.Cu") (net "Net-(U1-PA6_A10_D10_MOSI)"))
 (segment (start 162 77) (end 162 75.288428) (width 0.2) (layer "F.Cu") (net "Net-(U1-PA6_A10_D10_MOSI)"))
 (segment (start 157.06 76.56) (end 157.5 77) (width 0.2) (layer "F.Cu") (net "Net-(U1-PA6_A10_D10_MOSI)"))
 (segment (start 119.06 74.840101) (end 119.06 75.999899) (width 0.2) (layer "F.Cu") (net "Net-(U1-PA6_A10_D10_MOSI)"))
 (segment (start 152.110101 76.56) (end 157.06 76.56) (width 0.2) (layer "F.Cu") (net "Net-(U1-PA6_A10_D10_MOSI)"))
 (segment (start 132.700101 76.82) (end 133.480202 76.039899) (width 0.2) (layer "F.Cu") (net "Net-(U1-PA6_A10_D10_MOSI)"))
 (via (at 161.5 71) (size 0.6) (drill 0.3) (layers "F.Cu" "B.Cu") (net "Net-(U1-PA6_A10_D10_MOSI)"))
 (via (at 162 77) (size 0.6) (drill 0.3) (layers "F.Cu" "B.Cu") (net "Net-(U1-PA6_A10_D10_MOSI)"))
 (via (at 157.5 77) (size 0.6) (drill 0.3) (layers "F.Cu" "B.Cu") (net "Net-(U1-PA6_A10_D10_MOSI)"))
 (via (at 164.394214 72.894214) (size 0.6) (drill 0.3) (layers "F.Cu" "B.Cu") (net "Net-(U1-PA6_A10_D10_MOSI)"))
 (segment (start 157.5 77) (end 162 77) (width 0.2) (layer "B.Cu") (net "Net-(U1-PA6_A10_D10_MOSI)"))
 (segment (start 162.5 71) (end 161.5 71) (width 0.2) (layer "B.Cu") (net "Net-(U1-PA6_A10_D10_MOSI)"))
 (segment (start 164.394214 72.894214) (end 162.5 71) (width 0.2) (layer "B.Cu") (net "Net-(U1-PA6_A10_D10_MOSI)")))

